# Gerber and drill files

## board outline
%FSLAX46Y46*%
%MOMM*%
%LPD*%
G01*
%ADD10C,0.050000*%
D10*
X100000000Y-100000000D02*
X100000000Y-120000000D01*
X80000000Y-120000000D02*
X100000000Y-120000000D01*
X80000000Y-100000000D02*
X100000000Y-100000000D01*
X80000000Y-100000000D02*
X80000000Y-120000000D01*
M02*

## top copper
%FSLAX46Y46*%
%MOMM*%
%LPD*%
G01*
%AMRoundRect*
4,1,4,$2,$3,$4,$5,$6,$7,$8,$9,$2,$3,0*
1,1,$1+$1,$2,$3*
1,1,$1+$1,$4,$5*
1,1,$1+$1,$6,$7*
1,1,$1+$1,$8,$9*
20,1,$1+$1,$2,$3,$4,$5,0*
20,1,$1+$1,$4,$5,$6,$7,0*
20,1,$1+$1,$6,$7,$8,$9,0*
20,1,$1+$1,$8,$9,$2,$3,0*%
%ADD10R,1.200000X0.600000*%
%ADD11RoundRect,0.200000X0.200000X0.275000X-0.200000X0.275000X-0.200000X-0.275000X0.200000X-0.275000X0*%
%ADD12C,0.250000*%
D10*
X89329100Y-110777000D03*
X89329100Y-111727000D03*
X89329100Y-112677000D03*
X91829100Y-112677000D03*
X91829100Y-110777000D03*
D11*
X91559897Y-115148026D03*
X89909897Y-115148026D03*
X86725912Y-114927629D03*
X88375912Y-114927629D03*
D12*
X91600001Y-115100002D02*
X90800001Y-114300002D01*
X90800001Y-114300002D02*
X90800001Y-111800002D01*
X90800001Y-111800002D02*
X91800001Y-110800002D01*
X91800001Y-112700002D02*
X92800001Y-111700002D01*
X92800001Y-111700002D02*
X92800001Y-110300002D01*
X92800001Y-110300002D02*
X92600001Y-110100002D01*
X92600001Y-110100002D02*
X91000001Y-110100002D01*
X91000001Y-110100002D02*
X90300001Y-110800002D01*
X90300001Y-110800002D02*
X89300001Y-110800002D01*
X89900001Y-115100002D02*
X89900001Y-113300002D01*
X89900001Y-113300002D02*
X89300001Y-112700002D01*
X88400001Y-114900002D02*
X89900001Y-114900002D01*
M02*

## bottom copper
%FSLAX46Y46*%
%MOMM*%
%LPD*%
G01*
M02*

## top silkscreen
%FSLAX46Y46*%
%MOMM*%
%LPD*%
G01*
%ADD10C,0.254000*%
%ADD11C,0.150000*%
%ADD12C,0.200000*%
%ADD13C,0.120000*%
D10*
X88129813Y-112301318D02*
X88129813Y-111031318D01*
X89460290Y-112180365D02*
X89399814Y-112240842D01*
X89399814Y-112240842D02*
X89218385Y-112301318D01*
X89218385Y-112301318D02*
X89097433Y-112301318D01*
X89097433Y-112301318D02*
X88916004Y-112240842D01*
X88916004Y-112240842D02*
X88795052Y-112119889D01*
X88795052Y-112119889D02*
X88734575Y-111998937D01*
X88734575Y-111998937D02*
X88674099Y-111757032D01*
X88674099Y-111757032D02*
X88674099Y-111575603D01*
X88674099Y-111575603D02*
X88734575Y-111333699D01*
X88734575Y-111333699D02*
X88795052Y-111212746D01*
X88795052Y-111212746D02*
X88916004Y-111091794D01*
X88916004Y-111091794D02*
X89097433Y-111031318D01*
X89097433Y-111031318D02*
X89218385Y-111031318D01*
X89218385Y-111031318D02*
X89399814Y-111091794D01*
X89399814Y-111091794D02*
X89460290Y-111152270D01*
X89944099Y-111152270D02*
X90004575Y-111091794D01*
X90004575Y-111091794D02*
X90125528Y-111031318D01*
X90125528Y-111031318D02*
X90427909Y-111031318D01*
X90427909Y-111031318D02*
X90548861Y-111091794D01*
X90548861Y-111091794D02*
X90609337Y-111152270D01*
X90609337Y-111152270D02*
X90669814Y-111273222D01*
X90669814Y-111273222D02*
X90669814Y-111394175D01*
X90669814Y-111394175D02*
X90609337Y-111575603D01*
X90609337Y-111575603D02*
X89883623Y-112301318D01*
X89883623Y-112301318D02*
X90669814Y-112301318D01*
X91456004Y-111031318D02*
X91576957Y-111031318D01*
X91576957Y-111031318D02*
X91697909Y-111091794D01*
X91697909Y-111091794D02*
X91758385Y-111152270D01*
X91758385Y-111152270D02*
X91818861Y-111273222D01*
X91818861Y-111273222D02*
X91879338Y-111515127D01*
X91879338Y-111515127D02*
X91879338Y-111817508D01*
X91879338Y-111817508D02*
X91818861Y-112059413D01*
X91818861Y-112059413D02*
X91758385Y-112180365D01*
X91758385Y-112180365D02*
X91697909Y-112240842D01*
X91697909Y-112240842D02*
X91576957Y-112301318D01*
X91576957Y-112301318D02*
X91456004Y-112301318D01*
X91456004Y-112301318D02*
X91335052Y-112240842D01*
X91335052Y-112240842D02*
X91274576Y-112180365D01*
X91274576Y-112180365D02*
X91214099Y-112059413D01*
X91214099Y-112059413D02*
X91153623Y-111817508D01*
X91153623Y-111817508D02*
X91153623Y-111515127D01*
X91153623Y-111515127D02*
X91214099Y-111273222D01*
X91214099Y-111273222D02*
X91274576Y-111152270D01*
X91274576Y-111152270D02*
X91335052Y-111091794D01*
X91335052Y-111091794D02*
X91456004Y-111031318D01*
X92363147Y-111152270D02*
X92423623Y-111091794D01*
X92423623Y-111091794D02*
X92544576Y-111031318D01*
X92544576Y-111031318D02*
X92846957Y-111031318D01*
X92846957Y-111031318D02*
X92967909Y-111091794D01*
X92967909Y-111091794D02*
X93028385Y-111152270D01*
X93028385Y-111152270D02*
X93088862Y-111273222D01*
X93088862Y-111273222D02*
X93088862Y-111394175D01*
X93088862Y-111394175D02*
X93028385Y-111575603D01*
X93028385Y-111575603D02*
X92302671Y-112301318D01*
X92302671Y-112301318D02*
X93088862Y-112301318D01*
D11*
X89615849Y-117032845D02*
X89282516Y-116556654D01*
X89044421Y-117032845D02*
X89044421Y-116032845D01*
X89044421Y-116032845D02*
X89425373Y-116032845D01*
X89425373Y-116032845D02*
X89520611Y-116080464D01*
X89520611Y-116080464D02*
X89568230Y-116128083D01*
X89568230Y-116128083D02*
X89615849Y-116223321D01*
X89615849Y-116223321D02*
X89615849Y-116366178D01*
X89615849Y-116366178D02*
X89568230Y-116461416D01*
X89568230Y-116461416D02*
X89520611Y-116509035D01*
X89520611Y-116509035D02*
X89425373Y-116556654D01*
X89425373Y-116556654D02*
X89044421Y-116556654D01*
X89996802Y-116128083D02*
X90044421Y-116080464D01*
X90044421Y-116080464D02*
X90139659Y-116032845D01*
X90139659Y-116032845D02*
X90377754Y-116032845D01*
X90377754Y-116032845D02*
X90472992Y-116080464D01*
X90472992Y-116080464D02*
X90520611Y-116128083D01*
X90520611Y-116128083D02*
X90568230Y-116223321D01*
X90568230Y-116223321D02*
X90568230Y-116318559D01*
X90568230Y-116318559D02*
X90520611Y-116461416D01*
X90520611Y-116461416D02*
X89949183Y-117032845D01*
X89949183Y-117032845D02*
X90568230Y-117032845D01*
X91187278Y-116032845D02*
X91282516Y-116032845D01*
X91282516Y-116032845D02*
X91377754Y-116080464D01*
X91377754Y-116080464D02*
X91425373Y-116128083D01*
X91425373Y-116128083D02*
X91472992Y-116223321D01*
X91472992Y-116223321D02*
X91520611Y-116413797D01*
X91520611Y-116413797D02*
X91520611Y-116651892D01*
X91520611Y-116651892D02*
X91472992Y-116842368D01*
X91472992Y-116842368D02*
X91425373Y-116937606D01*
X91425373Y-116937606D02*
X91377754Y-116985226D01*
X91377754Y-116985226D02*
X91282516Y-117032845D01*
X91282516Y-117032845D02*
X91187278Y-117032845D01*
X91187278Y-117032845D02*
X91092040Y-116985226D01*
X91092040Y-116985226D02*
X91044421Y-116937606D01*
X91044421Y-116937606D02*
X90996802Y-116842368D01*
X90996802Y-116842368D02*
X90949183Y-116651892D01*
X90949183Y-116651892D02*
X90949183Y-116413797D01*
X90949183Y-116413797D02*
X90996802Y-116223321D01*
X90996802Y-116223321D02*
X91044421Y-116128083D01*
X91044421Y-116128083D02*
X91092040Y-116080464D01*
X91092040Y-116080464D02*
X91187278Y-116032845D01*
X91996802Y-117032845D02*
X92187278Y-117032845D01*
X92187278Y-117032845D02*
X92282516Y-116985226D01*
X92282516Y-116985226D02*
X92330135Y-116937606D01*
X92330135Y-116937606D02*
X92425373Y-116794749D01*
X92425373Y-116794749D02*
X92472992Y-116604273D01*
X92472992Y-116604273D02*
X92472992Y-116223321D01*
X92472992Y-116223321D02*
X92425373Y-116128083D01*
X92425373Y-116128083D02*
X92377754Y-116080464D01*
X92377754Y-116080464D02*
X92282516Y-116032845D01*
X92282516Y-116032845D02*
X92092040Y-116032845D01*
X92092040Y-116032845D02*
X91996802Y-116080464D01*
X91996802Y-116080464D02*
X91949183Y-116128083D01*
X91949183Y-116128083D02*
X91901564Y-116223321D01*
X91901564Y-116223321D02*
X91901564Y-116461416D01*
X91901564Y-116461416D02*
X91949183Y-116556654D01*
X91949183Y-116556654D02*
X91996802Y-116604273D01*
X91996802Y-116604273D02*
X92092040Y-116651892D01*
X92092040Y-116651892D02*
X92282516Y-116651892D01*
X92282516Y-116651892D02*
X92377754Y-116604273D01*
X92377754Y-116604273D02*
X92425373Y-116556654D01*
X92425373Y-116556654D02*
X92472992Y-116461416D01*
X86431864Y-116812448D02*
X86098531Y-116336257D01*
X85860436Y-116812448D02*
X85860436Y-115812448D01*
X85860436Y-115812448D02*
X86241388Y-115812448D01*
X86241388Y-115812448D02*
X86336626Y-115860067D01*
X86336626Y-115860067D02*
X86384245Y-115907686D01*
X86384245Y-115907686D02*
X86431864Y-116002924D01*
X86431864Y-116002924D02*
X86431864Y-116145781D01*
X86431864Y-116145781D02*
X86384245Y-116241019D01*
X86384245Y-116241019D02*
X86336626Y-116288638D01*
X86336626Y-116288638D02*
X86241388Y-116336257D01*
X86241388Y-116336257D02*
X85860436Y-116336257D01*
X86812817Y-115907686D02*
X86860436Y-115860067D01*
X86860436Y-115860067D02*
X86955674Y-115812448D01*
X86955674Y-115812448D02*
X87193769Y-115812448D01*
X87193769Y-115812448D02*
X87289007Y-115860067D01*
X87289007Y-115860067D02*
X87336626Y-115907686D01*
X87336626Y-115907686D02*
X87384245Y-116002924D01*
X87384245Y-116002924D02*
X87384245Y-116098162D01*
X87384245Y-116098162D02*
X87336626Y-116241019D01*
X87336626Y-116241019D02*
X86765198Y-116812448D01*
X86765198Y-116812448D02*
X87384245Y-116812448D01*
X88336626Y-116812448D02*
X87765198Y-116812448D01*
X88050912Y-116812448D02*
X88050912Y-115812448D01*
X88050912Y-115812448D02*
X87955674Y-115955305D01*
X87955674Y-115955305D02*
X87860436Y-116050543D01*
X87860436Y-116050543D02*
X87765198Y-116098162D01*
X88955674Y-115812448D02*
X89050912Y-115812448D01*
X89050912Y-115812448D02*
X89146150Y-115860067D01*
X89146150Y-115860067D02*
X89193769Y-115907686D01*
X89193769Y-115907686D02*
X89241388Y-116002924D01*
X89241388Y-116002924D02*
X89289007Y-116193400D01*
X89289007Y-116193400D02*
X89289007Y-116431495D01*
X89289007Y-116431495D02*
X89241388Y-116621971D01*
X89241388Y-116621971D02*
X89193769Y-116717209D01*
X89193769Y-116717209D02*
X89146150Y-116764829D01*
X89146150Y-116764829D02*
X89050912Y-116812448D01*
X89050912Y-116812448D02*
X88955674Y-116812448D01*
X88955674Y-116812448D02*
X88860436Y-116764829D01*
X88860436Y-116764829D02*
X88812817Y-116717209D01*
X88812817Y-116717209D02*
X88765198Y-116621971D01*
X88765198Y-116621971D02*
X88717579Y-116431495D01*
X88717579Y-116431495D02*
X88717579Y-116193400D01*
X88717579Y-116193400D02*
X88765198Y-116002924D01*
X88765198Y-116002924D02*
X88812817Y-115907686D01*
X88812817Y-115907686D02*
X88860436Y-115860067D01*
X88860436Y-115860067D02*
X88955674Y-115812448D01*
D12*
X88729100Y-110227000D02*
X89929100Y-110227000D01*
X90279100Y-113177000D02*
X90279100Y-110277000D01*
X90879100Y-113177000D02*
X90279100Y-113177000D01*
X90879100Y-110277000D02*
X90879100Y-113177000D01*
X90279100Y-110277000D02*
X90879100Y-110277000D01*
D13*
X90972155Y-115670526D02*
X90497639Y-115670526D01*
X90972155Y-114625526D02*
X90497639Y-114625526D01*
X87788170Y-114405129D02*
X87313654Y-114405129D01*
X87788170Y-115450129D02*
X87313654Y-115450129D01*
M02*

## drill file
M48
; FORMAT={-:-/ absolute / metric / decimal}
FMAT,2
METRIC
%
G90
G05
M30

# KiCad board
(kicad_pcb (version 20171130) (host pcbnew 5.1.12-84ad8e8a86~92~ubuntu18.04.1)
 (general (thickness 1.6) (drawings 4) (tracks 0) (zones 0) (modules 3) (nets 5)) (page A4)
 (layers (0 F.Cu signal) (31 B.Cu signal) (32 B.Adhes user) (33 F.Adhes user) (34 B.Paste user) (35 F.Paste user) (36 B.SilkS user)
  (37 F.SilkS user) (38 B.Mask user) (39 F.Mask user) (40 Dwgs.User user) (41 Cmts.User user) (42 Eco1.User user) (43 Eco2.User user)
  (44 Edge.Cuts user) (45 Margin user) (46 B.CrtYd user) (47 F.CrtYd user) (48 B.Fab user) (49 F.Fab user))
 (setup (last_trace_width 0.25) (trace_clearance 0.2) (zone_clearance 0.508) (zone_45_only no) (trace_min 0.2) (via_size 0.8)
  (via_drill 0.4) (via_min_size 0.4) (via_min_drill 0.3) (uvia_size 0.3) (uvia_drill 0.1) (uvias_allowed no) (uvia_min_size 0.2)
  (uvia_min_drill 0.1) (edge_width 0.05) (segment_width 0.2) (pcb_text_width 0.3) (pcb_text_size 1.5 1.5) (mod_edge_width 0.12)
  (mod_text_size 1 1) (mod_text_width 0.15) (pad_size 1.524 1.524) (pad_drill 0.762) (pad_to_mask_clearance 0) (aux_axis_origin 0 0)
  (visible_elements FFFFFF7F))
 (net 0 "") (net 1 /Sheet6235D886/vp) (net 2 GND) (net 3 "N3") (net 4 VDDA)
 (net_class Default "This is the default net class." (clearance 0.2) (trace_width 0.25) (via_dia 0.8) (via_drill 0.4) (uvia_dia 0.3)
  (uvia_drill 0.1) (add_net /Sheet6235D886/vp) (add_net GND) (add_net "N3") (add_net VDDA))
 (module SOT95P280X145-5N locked (layer F.Cu) (at 90.579100 111.727000)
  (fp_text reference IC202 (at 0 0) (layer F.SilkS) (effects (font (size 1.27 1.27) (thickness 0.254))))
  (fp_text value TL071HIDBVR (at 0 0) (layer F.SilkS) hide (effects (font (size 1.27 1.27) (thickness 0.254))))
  (fp_line (start -1.85 -1.5) (end -0.65 -1.5) (layer F.SilkS) (width 0.2))
  (fp_line (start -0.3 1.45) (end -0.3 -1.45) (layer F.SilkS) (width 0.2))
  (fp_line (start 0.3 1.45) (end -0.3 1.45) (layer F.SilkS) (width 0.2))
  (fp_line (start 0.3 -1.45) (end 0.3 1.45) (layer F.SilkS) (width 0.2))
  (fp_line (start -0.3 -1.45) (end 0.3 -1.45) (layer F.SilkS) (width 0.2))
  (pad 1 smd rect (at -1.25 -0.95 90.000000) (size 0.6 1.2) (layers F.Cu F.Mask F.Paste) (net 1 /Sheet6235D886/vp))
  (pad 2 smd rect (at -1.25 0 90.000000) (size 0.6 1.2) (layers F.Cu F.Mask F.Paste) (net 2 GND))
  (pad 3 smd rect (at -1.25 0.95 90.000000) (size 0.6 1.2) (layers F.Cu F.Mask F.Paste) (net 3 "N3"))
  (pad 4 smd rect (at 1.25 0.95 90.000000) (size 0.6 1.2) (layers F.Cu F.Mask F.Paste) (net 1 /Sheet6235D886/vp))
  (pad 5 smd rect (at 1.25 -0.95 90.000000) (size 0.6 1.2) (layers F.Cu F.Mask F.Paste) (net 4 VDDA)))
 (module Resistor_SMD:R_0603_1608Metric (layer F.Cu) (at 90.734897 115.148026 180.000000)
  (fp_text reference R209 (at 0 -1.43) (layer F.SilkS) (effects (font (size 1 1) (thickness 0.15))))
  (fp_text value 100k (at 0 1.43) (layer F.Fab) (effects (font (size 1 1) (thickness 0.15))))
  (fp_line (start -0.237258 -0.5225) (end 0.237258 -0.5225) (layer F.SilkS) (width 0.12))
  (fp_line (start -0.237258 0.5225) (end 0.237258 0.5225) (layer F.SilkS) (width 0.12))
  (pad 1 smd roundrect (at -0.825 0 180.000000) (size 0.8 0.95) (layers F.Cu F.Mask F.Paste) (roundrect_rratio 0.25) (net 4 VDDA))
  (pad 2 smd roundrect (at 0.825 0 180.000000) (size 0.8 0.95) (layers F.Cu F.Mask F.Paste) (roundrect_rratio 0.25) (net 3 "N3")))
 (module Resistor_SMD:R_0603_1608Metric (layer F.Cu) (at 87.550912 114.927629 180.000000)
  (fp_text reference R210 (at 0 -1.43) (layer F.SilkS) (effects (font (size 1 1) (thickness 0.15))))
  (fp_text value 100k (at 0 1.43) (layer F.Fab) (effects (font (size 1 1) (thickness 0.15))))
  (fp_line (start -0.237258 0.5225) (end 0.237258 0.5225) (layer F.SilkS) (width 0.12))
  (fp_line (start -0.237258 -0.5225) (end 0.237258 -0.5225) (layer F.SilkS) (width 0.12))
  (pad 2 smd roundrect (at 0.825 0 180.000000) (size 0.8 0.95) (layers F.Cu F.Mask F.Paste) (roundrect_rratio 0.25) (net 2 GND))
  (pad 1 smd roundrect (at -0.825 0 180.000000) (size 0.8 0.95) (layers F.Cu F.Mask F.Paste) (roundrect_rratio 0.25) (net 3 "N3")))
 (gr_line (start 100 100) (end 100 120) (layer Edge.Cuts) (width 0.05))
 (gr_line (start 80 120) (end 100 120) (layer Edge.Cuts) (width 0.05))
 (gr_line (start 80 100) (end 100 100) (layer Edge.Cuts) (width 0.05))
 (gr_line (start 80 100) (end 80 120) (layer Edge.Cuts) (width 0.05))
 (segment (start 91.600001 115.100002) (end 90.800001 114.300002) (width 0.250000) (layer F.Cu) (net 4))
 (segment (start 90.800001 114.300002) (end 90.800001 111.800002) (width 0.250000) (layer F.Cu) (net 4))
 (segment (start 90.800001 111.800002) (end 91.800001 110.800002) (width 0.250000) (layer F.Cu) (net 4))
 (segment (start 91.800001 112.700002) (end 92.800001 111.700002) (width 0.250000) (layer F.Cu) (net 1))
 (segment (start 92.800001 111.700002) (end 92.800001 110.300002) (width 0.250000) (layer F.Cu) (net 1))
 (segment (start 92.800001 110.300002) (end 92.600001 110.100002) (width 0.250000) (layer F.Cu) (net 1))
 (segment (start 92.600001 110.100002) (end 91.000001 110.100002) (width 0.250000) (layer F.Cu) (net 1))
 (segment (start 91.000001 110.100002) (end 90.300001 110.800002) (width 0.250000) (layer F.Cu) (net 1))
 (segment (start 90.300001 110.800002) (end 89.300001 110.800002) (width 0.250000) (layer F.Cu) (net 1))
 (segment (start 89.900001 115.100002) (end 89.900001 113.300002) (width 0.250000) (layer F.Cu) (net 3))
 (segment (start 89.900001 113.300002) (end 89.300001 112.700002) (width 0.250000) (layer F.Cu) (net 3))
 (segment (start 88.400001 114.900002) (end 89.900001 114.900002) (width 0.250000) (layer F.Cu) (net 3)))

